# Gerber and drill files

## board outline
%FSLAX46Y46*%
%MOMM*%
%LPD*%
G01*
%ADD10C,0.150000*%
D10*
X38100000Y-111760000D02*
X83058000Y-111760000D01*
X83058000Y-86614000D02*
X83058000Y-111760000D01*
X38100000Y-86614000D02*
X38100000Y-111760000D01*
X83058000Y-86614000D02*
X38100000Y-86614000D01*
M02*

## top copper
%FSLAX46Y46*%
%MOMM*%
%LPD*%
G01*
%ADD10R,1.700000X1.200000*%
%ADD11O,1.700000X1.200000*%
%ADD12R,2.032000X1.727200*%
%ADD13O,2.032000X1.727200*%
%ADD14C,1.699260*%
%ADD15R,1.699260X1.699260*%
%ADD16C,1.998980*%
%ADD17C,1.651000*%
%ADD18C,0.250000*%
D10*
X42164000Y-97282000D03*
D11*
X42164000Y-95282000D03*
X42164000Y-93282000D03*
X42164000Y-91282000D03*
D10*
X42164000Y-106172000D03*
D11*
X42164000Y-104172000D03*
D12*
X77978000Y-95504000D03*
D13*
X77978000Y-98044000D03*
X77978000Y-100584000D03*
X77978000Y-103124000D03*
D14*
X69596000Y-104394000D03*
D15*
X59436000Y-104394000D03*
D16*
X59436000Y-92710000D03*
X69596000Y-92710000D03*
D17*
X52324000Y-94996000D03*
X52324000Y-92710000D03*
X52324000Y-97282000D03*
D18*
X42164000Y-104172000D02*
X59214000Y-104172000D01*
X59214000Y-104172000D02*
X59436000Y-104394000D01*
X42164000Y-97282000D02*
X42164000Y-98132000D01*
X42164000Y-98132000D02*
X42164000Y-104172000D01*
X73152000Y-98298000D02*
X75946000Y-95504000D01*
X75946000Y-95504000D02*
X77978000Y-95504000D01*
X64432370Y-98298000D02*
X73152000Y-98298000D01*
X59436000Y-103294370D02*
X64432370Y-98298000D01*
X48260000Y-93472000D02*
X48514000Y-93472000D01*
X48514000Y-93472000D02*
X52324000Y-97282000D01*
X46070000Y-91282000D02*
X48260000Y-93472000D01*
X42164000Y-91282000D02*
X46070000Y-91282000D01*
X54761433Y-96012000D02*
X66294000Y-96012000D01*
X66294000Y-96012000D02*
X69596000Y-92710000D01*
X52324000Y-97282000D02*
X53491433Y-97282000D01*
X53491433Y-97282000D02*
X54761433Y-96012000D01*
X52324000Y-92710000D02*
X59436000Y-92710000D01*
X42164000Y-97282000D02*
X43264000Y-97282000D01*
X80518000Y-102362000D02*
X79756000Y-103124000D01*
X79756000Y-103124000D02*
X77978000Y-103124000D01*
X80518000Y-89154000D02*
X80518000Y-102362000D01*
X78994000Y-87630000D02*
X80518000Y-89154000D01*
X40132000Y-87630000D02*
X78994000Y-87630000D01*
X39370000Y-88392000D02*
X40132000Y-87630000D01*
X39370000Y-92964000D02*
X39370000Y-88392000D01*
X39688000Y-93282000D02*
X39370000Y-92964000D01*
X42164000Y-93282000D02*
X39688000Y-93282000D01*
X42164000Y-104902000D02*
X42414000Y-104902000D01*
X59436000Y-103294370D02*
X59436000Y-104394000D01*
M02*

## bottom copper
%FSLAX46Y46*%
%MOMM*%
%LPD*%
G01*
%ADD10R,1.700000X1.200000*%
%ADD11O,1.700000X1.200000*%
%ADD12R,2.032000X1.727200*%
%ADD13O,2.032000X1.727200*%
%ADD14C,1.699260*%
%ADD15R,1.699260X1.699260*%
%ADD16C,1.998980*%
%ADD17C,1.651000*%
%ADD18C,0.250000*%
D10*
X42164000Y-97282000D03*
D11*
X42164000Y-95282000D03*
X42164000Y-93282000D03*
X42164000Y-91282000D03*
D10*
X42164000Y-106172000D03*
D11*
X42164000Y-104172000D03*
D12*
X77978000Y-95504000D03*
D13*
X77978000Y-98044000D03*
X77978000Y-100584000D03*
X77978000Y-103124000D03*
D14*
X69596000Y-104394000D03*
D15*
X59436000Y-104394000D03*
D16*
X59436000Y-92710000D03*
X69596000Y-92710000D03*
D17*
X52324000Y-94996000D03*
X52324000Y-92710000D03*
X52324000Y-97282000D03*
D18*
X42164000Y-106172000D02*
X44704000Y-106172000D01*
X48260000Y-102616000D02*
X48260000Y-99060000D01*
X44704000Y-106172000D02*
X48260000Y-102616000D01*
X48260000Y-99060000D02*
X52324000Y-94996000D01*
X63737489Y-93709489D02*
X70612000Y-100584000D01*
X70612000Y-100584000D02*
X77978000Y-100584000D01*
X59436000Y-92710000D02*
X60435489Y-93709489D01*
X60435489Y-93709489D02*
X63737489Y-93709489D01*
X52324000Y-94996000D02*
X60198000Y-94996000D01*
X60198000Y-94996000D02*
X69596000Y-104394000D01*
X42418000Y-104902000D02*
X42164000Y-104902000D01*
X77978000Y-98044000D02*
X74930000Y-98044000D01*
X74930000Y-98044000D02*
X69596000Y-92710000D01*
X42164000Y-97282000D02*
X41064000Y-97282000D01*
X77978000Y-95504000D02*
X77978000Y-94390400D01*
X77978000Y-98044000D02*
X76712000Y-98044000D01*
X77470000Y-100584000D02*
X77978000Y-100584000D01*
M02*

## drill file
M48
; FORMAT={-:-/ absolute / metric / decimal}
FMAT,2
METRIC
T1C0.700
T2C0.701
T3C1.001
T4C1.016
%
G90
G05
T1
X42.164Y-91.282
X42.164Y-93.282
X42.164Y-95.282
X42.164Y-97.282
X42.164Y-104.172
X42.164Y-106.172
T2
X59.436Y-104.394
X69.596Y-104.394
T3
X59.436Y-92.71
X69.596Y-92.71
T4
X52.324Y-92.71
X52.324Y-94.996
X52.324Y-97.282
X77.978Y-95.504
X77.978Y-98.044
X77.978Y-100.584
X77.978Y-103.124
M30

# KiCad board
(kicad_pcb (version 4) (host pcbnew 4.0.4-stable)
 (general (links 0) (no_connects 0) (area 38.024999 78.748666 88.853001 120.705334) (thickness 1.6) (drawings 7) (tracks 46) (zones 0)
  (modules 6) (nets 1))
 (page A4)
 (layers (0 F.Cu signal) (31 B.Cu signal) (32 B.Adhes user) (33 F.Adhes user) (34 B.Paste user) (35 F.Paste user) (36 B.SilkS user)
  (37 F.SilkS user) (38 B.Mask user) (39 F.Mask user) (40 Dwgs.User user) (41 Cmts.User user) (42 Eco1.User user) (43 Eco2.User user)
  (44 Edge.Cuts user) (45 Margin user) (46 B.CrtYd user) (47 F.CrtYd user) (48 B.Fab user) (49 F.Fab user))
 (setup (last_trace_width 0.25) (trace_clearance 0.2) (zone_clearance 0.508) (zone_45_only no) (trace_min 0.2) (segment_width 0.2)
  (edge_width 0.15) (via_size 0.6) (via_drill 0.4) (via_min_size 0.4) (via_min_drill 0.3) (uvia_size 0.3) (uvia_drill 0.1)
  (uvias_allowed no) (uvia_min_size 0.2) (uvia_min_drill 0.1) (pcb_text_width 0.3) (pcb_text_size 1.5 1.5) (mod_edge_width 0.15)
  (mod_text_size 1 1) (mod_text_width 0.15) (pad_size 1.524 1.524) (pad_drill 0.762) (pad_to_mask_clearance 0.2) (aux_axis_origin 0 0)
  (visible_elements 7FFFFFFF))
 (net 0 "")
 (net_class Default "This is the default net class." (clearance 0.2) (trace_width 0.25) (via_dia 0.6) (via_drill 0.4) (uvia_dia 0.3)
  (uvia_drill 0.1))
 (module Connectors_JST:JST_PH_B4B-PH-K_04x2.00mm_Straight (layer F.Cu) (at 42.164 97.282 90)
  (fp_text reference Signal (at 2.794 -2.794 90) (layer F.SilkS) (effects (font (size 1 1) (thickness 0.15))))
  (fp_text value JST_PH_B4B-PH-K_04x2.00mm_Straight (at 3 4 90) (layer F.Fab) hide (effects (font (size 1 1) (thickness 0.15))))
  (pad 1 thru_hole rect (at 0 0 90) (size 1.2 1.7) (drill 0.7) (layers *.Cu *.Mask))
  (pad 2 thru_hole oval (at 2 0 90) (size 1.2 1.7) (drill 0.7) (layers *.Cu *.Mask))
  (pad 3 thru_hole oval (at 4 0 90) (size 1.2 1.7) (drill 0.7) (layers *.Cu *.Mask))
  (pad 4 thru_hole oval (at 6 0 90) (size 1.2 1.7) (drill 0.7) (layers *.Cu *.Mask)))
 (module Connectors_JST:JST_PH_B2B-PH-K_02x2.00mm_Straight (layer F.Cu) (at 42.164 106.172 90)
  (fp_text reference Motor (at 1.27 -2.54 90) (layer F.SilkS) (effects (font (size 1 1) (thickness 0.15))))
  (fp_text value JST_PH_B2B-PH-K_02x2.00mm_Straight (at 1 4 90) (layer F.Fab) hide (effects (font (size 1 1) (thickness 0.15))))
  (pad 1 thru_hole rect (at 0 0 90) (size 1.2 1.7) (drill 0.7) (layers *.Cu *.Mask))
  (pad 2 thru_hole oval (at 2 0 90) (size 1.2 1.7) (drill 0.7) (layers *.Cu *.Mask)))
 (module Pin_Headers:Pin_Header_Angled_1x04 (layer F.Cu) (at 77.978 95.504)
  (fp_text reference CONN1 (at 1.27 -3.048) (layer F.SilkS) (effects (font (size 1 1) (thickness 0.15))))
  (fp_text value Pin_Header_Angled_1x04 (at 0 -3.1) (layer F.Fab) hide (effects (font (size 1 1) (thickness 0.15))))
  (pad 1 thru_hole rect (at 0 0) (size 2.032 1.7272) (drill 1.016) (layers *.Cu *.Mask))
  (pad 2 thru_hole oval (at 0 2.54) (size 2.032 1.7272) (drill 1.016) (layers *.Cu *.Mask))
  (pad 3 thru_hole oval (at 0 5.08) (size 2.032 1.7272) (drill 1.016) (layers *.Cu *.Mask))
  (pad 4 thru_hole oval (at 0 7.62) (size 2.032 1.7272) (drill 1.016) (layers *.Cu *.Mask)))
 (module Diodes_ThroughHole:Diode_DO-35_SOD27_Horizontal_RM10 (layer F.Cu) (at 59.43548 104.39654)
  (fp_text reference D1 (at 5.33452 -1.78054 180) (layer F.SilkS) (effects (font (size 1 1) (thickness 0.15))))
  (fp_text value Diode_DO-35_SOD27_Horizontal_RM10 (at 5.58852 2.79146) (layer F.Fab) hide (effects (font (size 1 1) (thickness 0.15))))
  (pad 2 thru_hole circle (at 10.16052 -0.00254 180) (size 1.69926 1.69926) (drill 0.70104) (layers *.Cu *.Mask))
  (pad 1 thru_hole rect (at 0.00052 -0.00254 180) (size 1.69926 1.69926) (drill 0.70104) (layers *.Cu *.Mask)))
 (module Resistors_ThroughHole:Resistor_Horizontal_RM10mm (layer F.Cu) (at 59.436 92.71)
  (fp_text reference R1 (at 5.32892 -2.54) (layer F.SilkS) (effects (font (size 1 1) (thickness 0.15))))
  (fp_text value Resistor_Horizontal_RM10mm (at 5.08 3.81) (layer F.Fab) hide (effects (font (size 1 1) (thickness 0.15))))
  (pad 1 thru_hole circle (at 0 0) (size 1.99898 1.99898) (drill 1.00076) (layers *.Cu *.SilkS *.Mask))
  (pad 2 thru_hole circle (at 10.16 0) (size 1.99898 1.99898) (drill 1.00076) (layers *.Cu *.SilkS *.Mask)))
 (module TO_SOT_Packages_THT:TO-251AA (layer F.Cu) (at 52.324 97.282 90)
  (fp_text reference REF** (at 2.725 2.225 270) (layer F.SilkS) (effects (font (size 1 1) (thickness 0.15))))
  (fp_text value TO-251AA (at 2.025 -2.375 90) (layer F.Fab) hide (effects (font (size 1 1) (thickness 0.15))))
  (pad 2 thru_hole circle (at 2.286 0 270) (size 1.651 1.651) (drill 1.016) (layers *.Cu *.Mask))
  (pad 3 thru_hole circle (at 4.572 0 270) (size 1.651 1.651) (drill 1.016) (layers *.Cu *.Mask))
  (pad 1 thru_hole circle (at 0 0 270) (size 1.651 1.651) (drill 1.016) (layers *.Cu *.Mask)))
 (gr_line (start 38.1 111.76) (end 83.058 111.76) (layer Edge.Cuts) (width 0.15))
 (gr_line (start 83.058 86.614) (end 83.058 111.76) (layer Edge.Cuts) (width 0.15))
 (gr_line (start 38.1 86.614) (end 38.1 111.76) (layer Edge.Cuts) (width 0.15))
 (gr_line (start 83.058 86.614) (end 38.1 86.614) (layer Edge.Cuts) (width 0.15))
 (segment (start 42.164 106.172) (end 44.704 106.172) (width 0.25) (layer B.Cu) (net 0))
 (segment (start 48.26 102.616) (end 48.26 99.06) (width 0.25) (layer B.Cu) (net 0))
 (segment (start 44.704 106.172) (end 48.26 102.616) (width 0.25) (layer B.Cu) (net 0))
 (segment (start 48.26 99.06) (end 52.324 94.996) (width 0.25) (layer B.Cu) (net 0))
 (segment (start 42.164 104.172) (end 59.214 104.172) (width 0.25) (layer F.Cu) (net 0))
 (segment (start 59.214 104.172) (end 59.436 104.394) (width 0.25) (layer F.Cu) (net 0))
 (segment (start 42.164 97.282) (end 42.164 98.132) (width 0.25) (layer F.Cu) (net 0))
 (segment (start 42.164 98.132) (end 42.164 104.172) (width 0.25) (layer F.Cu) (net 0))
 (segment (start 73.152 98.298) (end 75.946 95.504) (width 0.25) (layer F.Cu) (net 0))
 (segment (start 75.946 95.504) (end 77.978 95.504) (width 0.25) (layer F.Cu) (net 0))
 (segment (start 64.43237 98.298) (end 73.152 98.298) (width 0.25) (layer F.Cu) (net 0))
 (segment (start 59.436 103.29437) (end 64.43237 98.298) (width 0.25) (layer F.Cu) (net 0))
 (segment (start 63.737489 93.709489) (end 70.612 100.584) (width 0.25) (layer B.Cu) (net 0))
 (segment (start 70.612 100.584) (end 77.978 100.584) (width 0.25) (layer B.Cu) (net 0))
 (segment (start 59.436 92.71) (end 60.435489 93.709489) (width 0.25) (layer B.Cu) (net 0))
 (segment (start 60.435489 93.709489) (end 63.737489 93.709489) (width 0.25) (layer B.Cu) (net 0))
 (segment (start 52.324 94.996) (end 60.198 94.996) (width 0.25) (layer B.Cu) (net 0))
 (segment (start 60.198 94.996) (end 69.596 104.394) (width 0.25) (layer B.Cu) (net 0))
 (segment (start 48.26 93.472) (end 48.514 93.472) (width 0.25) (layer F.Cu) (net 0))
 (segment (start 48.514 93.472) (end 52.324 97.282) (width 0.25) (layer F.Cu) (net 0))
 (segment (start 46.07 91.282) (end 48.26 93.472) (width 0.25) (layer F.Cu) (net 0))
 (segment (start 42.164 91.282) (end 46.07 91.282) (width 0.25) (layer F.Cu) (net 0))
 (segment (start 42.418 104.902) (end 42.164 104.902) (width 0.25) (layer B.Cu) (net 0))
 (segment (start 77.978 98.044) (end 74.93 98.044) (width 0.25) (layer B.Cu) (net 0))
 (segment (start 74.93 98.044) (end 69.596 92.71) (width 0.25) (layer B.Cu) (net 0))
 (segment (start 54.761433 96.012) (end 66.294 96.012) (width 0.25) (layer F.Cu) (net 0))
 (segment (start 66.294 96.012) (end 69.596 92.71) (width 0.25) (layer F.Cu) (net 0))
 (segment (start 52.324 97.282) (end 53.491433 97.282) (width 0.25) (layer F.Cu) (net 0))
 (segment (start 53.491433 97.282) (end 54.761433 96.012) (width 0.25) (layer F.Cu) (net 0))
 (segment (start 52.324 92.71) (end 59.436 92.71) (width 0.25) (layer F.Cu) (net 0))
 (segment (start 42.164 97.282) (end 43.264 97.282) (width 0.25) (layer F.Cu) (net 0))
 (segment (start 42.164 97.282) (end 41.064 97.282) (width 0.25) (layer B.Cu) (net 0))
 (segment (start 80.518 102.362) (end 79.756 103.124) (width 0.25) (layer F.Cu) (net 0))
 (segment (start 79.756 103.124) (end 77.978 103.124) (width 0.25) (layer F.Cu) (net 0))
 (segment (start 80.518 89.154) (end 80.518 102.362) (width 0.25) (layer F.Cu) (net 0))
 (segment (start 78.994 87.63) (end 80.518 89.154) (width 0.25) (layer F.Cu) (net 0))
 (segment (start 40.132 87.63) (end 78.994 87.63) (width 0.25) (layer F.Cu) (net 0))
 (segment (start 39.37 88.392) (end 40.132 87.63) (width 0.25) (layer F.Cu) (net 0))
 (segment (start 39.37 92.964) (end 39.37 88.392) (width 0.25) (layer F.Cu) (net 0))
 (segment (start 39.688 93.282) (end 39.37 92.964) (width 0.25) (layer F.Cu) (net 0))
 (segment (start 42.164 93.282) (end 39.688 93.282) (width 0.25) (layer F.Cu) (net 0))
 (segment (start 77.978 95.504) (end 77.978 94.3904) (width 0.25) (layer B.Cu) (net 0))
 (segment (start 77.978 98.044) (end 76.712 98.044) (width 0.25) (layer B.Cu) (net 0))
 (segment (start 77.47 100.584) (end 77.978 100.584) (width 0.25) (layer B.Cu) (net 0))
 (segment (start 42.164 104.902) (end 42.414 104.902) (width 0.25) (layer F.Cu) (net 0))
 (segment (start 59.436 103.29437) (end 59.436 104.394) (width 0.25) (layer F.Cu) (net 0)))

